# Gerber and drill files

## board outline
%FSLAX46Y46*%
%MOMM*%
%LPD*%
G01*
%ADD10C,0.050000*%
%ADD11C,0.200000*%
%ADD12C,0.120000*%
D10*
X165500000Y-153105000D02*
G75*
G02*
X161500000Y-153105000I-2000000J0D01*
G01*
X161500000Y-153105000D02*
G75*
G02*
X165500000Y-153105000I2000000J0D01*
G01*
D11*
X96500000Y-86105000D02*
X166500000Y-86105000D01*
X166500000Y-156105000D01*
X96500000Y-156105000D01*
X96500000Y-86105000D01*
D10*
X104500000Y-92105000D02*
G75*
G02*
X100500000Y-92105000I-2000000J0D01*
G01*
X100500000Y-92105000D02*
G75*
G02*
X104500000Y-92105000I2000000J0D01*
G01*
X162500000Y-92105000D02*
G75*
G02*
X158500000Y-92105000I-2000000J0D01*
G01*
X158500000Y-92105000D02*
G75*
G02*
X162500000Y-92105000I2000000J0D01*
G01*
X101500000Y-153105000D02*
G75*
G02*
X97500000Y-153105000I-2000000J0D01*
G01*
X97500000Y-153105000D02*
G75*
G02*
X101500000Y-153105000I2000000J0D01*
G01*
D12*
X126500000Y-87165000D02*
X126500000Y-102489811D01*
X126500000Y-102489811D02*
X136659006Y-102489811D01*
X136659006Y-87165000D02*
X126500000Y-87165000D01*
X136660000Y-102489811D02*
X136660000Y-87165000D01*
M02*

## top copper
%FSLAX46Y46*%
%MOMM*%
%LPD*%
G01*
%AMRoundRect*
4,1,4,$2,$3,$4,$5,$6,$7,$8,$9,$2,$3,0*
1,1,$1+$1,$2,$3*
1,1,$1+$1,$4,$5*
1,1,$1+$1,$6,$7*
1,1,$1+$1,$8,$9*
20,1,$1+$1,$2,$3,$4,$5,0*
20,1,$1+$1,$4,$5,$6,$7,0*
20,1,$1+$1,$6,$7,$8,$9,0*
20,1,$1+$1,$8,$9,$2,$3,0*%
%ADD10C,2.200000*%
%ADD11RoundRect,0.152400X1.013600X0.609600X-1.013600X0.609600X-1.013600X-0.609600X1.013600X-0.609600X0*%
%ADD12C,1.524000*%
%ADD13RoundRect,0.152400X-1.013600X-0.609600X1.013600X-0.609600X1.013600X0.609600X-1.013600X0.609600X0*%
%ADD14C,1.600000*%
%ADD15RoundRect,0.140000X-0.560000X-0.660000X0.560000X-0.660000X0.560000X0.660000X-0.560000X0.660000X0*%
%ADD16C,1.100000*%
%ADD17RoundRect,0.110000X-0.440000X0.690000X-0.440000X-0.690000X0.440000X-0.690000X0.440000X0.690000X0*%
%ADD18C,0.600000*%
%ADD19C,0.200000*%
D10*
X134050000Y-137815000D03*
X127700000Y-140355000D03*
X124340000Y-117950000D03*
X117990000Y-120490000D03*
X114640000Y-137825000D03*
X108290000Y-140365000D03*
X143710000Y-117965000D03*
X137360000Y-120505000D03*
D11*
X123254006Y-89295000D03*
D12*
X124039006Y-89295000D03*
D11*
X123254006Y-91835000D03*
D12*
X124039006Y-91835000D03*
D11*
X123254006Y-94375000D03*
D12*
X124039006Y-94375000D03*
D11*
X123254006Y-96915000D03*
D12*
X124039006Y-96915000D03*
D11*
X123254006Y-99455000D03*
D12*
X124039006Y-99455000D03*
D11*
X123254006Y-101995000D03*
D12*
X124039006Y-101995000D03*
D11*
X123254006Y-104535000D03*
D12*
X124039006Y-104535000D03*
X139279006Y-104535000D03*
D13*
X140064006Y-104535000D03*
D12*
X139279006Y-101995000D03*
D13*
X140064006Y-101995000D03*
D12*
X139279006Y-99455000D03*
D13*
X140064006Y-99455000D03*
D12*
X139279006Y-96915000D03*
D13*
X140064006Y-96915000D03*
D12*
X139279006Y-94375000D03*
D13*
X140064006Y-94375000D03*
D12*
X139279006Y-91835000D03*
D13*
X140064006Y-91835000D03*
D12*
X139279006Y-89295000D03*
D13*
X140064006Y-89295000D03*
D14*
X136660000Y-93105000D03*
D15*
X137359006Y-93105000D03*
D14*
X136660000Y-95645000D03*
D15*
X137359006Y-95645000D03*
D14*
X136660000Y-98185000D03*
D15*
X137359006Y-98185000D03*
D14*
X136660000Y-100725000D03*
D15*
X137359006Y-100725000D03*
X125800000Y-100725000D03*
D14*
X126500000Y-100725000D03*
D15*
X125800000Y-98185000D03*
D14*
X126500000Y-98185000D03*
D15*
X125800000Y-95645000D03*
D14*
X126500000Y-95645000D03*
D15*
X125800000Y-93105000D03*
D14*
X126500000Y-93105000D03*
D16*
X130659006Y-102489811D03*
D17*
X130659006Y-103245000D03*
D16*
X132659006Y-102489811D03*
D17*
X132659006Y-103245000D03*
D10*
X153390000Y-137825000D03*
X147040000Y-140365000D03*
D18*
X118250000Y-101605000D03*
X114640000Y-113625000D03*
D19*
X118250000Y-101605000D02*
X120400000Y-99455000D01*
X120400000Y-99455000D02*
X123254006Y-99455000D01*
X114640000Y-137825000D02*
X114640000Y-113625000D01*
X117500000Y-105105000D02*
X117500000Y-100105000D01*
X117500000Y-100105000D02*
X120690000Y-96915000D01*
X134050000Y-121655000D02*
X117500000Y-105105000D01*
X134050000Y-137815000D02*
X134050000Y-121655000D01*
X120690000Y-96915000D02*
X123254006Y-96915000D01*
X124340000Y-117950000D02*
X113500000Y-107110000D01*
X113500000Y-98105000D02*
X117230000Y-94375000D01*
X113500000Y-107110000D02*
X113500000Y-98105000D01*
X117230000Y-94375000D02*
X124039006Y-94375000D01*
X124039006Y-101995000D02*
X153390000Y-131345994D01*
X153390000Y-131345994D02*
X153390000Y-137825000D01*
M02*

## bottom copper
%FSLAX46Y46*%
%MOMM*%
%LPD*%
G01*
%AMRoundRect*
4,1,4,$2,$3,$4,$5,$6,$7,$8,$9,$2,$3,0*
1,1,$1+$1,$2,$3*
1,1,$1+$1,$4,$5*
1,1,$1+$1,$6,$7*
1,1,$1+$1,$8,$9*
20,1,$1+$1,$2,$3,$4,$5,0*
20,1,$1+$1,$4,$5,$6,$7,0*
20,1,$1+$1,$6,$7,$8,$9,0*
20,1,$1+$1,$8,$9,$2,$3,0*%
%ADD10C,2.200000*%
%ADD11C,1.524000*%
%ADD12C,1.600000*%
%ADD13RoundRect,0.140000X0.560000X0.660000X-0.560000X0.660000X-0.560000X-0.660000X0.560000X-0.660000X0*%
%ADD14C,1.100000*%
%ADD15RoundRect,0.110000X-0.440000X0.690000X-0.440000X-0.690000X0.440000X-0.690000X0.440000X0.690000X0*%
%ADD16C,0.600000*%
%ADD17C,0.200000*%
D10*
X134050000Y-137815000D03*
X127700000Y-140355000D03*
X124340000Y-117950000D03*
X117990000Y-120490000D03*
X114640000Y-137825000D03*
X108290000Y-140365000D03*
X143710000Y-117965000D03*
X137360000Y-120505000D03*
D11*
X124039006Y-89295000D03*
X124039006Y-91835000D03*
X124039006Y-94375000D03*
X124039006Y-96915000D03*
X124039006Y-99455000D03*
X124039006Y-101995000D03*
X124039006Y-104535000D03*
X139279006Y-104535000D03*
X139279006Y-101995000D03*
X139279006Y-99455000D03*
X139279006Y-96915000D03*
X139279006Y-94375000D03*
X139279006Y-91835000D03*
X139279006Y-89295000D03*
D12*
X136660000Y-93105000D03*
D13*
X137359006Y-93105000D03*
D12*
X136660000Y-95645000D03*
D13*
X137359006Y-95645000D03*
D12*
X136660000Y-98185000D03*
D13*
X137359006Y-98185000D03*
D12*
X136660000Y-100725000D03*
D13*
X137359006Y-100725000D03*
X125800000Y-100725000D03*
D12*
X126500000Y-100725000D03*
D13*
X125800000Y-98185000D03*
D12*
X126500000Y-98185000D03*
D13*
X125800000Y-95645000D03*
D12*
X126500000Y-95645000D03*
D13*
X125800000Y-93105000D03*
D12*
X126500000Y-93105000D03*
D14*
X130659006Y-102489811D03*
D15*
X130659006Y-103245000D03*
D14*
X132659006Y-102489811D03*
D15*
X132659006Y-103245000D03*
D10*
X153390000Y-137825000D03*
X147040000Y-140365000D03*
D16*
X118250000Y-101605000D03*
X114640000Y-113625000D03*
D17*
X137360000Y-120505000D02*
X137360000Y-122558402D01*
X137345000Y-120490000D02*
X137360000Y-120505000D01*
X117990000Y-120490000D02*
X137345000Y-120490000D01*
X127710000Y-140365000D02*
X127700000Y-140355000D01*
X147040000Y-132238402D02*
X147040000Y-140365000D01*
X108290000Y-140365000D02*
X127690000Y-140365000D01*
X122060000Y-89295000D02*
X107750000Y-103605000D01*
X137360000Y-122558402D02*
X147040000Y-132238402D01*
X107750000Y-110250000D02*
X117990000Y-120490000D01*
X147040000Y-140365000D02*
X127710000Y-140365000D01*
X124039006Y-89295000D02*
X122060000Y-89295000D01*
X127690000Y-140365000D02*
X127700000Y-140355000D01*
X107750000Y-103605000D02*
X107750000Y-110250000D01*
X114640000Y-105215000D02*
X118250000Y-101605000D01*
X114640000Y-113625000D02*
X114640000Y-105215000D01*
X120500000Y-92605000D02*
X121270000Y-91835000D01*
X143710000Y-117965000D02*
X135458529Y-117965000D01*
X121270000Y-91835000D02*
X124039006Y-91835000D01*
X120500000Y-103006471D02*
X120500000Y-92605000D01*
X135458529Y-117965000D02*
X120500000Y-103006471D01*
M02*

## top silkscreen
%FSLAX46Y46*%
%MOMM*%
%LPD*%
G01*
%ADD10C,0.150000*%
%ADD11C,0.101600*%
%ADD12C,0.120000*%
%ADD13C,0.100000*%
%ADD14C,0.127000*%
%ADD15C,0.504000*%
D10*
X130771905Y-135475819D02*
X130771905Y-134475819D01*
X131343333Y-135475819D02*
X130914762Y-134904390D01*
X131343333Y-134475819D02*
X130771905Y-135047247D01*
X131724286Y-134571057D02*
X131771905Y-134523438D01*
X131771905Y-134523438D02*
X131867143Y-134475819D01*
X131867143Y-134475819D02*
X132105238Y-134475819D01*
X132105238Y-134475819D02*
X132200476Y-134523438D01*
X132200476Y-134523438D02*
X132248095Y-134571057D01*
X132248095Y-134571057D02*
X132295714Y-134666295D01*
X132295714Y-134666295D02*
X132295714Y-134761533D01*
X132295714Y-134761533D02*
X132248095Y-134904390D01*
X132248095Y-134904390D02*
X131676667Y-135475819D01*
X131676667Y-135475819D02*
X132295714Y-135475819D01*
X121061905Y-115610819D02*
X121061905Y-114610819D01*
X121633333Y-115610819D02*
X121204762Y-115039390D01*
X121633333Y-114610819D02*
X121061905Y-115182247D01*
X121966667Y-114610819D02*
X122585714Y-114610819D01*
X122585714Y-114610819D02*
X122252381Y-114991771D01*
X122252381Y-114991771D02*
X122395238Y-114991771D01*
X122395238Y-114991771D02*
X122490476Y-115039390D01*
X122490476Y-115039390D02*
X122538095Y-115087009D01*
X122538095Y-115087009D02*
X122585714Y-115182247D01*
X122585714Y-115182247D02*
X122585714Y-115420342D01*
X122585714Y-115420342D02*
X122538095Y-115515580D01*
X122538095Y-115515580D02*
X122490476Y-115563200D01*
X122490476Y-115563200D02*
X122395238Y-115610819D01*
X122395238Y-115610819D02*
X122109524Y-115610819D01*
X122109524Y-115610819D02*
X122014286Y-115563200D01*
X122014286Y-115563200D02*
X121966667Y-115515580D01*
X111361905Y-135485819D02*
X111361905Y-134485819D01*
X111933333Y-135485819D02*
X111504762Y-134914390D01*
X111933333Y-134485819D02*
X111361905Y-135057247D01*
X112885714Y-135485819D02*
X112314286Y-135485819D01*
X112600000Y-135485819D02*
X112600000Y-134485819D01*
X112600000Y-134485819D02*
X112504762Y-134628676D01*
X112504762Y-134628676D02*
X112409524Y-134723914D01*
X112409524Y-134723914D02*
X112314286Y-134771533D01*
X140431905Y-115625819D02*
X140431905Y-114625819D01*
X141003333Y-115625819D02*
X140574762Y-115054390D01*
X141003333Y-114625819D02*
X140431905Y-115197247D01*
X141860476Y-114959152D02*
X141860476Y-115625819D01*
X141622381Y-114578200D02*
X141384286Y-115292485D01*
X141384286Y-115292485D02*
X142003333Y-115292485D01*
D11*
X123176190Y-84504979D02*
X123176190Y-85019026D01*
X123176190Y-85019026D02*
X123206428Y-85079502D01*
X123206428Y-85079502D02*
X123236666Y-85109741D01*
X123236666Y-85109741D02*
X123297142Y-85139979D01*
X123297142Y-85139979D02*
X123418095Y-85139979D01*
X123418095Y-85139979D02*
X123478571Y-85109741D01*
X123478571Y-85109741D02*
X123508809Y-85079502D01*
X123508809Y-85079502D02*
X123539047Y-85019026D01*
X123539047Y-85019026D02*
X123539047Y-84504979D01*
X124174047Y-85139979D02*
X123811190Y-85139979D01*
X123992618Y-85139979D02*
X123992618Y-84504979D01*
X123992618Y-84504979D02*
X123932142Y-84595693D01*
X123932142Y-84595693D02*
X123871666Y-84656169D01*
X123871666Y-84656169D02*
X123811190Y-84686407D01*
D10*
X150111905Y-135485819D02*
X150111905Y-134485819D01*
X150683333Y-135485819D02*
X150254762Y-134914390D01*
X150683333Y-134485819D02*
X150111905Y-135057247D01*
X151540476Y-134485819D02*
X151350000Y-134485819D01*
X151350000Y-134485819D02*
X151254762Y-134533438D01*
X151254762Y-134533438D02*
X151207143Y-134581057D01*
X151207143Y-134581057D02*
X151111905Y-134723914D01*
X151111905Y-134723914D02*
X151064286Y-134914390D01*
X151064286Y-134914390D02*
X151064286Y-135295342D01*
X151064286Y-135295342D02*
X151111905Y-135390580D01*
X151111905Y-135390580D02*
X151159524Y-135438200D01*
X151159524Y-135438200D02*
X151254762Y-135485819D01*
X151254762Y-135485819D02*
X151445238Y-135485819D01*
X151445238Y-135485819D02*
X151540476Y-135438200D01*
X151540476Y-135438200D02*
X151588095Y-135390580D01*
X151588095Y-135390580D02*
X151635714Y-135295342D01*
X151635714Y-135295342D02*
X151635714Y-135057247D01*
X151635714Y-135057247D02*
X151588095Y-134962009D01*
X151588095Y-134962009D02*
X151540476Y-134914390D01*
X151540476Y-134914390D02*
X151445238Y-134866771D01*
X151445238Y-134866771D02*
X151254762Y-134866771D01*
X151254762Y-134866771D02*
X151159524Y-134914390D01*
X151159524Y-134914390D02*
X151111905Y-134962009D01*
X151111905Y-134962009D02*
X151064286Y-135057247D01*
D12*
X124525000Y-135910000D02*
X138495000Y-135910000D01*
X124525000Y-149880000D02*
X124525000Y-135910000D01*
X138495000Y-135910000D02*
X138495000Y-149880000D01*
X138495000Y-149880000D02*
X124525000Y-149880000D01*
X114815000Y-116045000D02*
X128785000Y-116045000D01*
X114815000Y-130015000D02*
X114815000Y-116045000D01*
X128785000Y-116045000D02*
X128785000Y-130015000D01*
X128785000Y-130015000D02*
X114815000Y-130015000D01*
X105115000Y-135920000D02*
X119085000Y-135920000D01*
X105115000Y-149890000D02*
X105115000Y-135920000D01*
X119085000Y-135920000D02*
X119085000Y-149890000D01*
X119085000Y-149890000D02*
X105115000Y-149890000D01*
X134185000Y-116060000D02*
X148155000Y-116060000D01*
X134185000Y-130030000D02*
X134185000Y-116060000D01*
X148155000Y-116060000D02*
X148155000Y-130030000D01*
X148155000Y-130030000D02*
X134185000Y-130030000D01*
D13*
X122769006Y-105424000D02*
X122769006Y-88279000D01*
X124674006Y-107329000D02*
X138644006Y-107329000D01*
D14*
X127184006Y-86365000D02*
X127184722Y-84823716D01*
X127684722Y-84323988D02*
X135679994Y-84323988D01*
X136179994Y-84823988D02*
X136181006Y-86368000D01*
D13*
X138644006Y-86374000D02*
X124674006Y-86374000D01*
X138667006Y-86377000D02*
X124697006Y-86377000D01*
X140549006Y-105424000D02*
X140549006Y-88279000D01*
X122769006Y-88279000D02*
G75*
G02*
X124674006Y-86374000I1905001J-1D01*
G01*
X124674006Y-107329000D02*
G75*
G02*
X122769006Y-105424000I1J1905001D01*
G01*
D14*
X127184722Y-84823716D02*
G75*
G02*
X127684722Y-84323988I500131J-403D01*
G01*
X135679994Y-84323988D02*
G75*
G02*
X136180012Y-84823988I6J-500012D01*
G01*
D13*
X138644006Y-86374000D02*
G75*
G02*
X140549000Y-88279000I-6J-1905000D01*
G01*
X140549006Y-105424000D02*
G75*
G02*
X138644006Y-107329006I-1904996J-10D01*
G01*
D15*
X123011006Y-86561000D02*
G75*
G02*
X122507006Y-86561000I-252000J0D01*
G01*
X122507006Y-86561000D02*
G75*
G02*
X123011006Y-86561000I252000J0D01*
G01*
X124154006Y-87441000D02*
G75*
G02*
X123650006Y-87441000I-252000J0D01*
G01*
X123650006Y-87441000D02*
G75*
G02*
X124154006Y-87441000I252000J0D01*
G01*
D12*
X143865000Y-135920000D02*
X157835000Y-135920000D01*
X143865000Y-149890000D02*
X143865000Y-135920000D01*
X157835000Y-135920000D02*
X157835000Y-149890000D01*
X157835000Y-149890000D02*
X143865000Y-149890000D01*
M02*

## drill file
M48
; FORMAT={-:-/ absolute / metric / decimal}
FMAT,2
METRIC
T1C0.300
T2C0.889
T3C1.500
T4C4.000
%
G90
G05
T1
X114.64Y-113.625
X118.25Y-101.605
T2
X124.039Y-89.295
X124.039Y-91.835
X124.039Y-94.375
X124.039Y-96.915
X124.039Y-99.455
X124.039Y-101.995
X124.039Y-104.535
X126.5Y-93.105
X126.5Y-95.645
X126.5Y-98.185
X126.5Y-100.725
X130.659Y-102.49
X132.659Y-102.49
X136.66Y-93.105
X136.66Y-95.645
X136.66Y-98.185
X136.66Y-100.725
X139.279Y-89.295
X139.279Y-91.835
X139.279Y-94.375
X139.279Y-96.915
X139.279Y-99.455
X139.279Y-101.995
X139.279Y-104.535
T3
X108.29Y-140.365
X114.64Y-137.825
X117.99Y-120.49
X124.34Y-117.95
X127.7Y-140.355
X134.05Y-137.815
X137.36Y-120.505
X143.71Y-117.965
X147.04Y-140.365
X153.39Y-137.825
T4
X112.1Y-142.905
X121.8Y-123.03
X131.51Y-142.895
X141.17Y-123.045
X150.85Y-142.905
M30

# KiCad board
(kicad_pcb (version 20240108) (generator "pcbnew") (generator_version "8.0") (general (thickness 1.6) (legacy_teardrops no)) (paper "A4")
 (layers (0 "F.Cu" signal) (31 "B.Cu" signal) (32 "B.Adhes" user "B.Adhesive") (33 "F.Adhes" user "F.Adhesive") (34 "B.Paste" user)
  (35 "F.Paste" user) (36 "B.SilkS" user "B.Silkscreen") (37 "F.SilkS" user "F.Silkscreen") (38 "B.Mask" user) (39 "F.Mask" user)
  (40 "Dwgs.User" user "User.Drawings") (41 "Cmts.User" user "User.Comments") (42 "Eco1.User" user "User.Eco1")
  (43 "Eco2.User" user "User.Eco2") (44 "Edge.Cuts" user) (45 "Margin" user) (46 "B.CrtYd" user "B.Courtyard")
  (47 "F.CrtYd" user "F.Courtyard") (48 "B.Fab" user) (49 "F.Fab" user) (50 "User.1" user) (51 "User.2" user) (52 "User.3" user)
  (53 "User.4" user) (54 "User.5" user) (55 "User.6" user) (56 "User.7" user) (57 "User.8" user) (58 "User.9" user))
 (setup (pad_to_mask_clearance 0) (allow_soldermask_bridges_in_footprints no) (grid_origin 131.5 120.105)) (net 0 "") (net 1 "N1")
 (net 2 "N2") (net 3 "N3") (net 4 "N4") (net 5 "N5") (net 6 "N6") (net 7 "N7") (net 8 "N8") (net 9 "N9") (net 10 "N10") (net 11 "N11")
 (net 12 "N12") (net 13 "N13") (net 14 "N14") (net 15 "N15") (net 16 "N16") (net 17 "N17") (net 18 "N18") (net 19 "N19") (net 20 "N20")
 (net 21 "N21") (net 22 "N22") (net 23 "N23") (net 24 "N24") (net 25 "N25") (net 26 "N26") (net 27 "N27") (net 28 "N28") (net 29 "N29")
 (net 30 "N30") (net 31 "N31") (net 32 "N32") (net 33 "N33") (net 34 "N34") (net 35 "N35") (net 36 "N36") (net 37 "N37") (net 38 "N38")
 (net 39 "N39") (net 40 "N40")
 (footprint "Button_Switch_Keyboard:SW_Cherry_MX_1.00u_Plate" (layer "F.Cu") (at 134.05 137.815)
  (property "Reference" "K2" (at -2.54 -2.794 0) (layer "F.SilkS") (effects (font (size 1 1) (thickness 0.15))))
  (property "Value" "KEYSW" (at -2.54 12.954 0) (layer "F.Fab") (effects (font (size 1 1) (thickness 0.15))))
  (fp_line (start -9.525 -1.905) (end 4.445 -1.905) (stroke (width 0.12) (type solid)) (layer "F.SilkS"))
  (fp_line (start -9.525 12.065) (end -9.525 -1.905) (stroke (width 0.12) (type solid)) (layer "F.SilkS"))
  (fp_line (start 4.445 -1.905) (end 4.445 12.065) (stroke (width 0.12) (type solid)) (layer "F.SilkS"))
  (fp_line (start 4.445 12.065) (end -9.525 12.065) (stroke (width 0.12) (type solid)) (layer "F.SilkS"))
  (pad "" np_thru_hole circle (at -2.54 5.08) (size 4 4) (drill 4) (layers "*.Cu" "*.Mask"))
  (pad "1" thru_hole circle (at 0 0) (size 2.2 2.2) (drill 1.5) (layers "*.Cu" "*.Mask") (remove_unused_layers no) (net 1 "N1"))
  (pad "2" thru_hole circle (at -6.35 2.54) (size 2.2 2.2) (drill 1.5) (layers "*.Cu" "*.Mask") (remove_unused_layers no) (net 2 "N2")))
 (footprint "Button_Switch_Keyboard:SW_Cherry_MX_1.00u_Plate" (layer "F.Cu") (at 124.34 117.95)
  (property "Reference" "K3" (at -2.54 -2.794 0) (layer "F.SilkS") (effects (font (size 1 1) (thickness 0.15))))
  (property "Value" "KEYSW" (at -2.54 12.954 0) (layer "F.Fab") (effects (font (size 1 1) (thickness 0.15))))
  (fp_line (start -9.525 -1.905) (end 4.445 -1.905) (stroke (width 0.12) (type solid)) (layer "F.SilkS"))
  (fp_line (start -9.525 12.065) (end -9.525 -1.905) (stroke (width 0.12) (type solid)) (layer "F.SilkS"))
  (fp_line (start 4.445 -1.905) (end 4.445 12.065) (stroke (width 0.12) (type solid)) (layer "F.SilkS"))
  (fp_line (start 4.445 12.065) (end -9.525 12.065) (stroke (width 0.12) (type solid)) (layer "F.SilkS"))
  (pad "" np_thru_hole circle (at -2.54 5.08) (size 4 4) (drill 4) (layers "*.Cu" "*.Mask"))
  (pad "1" thru_hole circle (at 0 0) (size 2.2 2.2) (drill 1.5) (layers "*.Cu" "*.Mask") (remove_unused_layers no) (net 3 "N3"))
  (pad "2" thru_hole circle (at -6.35 2.54) (size 2.2 2.2) (drill 1.5) (layers "*.Cu" "*.Mask") (remove_unused_layers no) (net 2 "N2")))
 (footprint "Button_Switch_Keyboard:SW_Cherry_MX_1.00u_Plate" (layer "F.Cu") (at 114.64 137.825)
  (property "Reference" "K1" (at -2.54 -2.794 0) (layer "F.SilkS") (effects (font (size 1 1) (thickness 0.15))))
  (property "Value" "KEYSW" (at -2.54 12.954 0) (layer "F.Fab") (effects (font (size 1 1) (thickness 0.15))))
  (fp_line (start -9.525 -1.905) (end 4.445 -1.905) (stroke (width 0.12) (type solid)) (layer "F.SilkS"))
  (fp_line (start -9.525 12.065) (end -9.525 -1.905) (stroke (width 0.12) (type solid)) (layer "F.SilkS"))
  (fp_line (start 4.445 -1.905) (end 4.445 12.065) (stroke (width 0.12) (type solid)) (layer "F.SilkS"))
  (fp_line (start 4.445 12.065) (end -9.525 12.065) (stroke (width 0.12) (type solid)) (layer "F.SilkS"))
  (pad "" np_thru_hole circle (at -2.54 5.08) (size 4 4) (drill 4) (layers "*.Cu" "*.Mask"))
  (pad "1" thru_hole circle (at 0 0) (size 2.2 2.2) (drill 1.5) (layers "*.Cu" "*.Mask") (remove_unused_layers no) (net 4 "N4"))
  (pad "2" thru_hole circle (at -6.35 2.54) (size 2.2 2.2) (drill 1.5) (layers "*.Cu" "*.Mask") (remove_unused_layers no) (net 2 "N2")))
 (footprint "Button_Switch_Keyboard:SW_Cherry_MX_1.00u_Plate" (layer "F.Cu") (at 143.71 117.965)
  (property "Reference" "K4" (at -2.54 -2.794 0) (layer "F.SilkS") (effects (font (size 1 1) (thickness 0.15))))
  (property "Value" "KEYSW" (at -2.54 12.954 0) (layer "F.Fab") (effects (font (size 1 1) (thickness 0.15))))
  (fp_line (start -9.525 -1.905) (end 4.445 -1.905) (stroke (width 0.12) (type solid)) (layer "F.SilkS"))
  (fp_line (start -9.525 12.065) (end -9.525 -1.905) (stroke (width 0.12) (type solid)) (layer "F.SilkS"))
  (fp_line (start 4.445 -1.905) (end 4.445 12.065) (stroke (width 0.12) (type solid)) (layer "F.SilkS"))
  (fp_line (start 4.445 12.065) (end -9.525 12.065) (stroke (width 0.12) (type solid)) (layer "F.SilkS"))
  (pad "" np_thru_hole circle (at -2.54 5.08) (size 4 4) (drill 4) (layers "*.Cu" "*.Mask"))
  (pad "1" thru_hole circle (at 0 0) (size 2.2 2.2) (drill 1.5) (layers "*.Cu" "*.Mask") (remove_unused_layers no) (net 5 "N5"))
  (pad "2" thru_hole circle (at -6.35 2.54) (size 2.2 2.2) (drill 1.5) (layers "*.Cu" "*.Mask") (remove_unused_layers no) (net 2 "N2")))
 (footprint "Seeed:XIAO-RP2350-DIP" (layer "F.Cu") (at 131.66 96.8515)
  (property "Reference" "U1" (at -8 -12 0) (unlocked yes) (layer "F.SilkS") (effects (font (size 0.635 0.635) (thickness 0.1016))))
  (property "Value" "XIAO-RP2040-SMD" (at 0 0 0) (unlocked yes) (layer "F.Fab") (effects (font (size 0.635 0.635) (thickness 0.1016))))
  (fp_line (start -8.890994 8.5725) (end -8.890994 -8.5725) (stroke (width 0.1) (type solid)) (layer "F.SilkS"))
  (fp_line (start -6.985994 10.4775) (end 6.984006 10.4775) (stroke (width 0.1) (type solid)) (layer "F.SilkS"))
  (fp_line (start -4.475994 -10.4865) (end -4.475278 -12.027784) (stroke (width 0.127) (type solid)) (layer "F.SilkS"))
  (fp_line (start -3.975278 -12.527512) (end 4.019994 -12.527512) (stroke (width 0.127) (type solid)) (layer "F.SilkS"))
  (fp_line (start 4.519994 -12.027512) (end 4.521006 -10.4835) (stroke (width 0.127) (type solid)) (layer "F.SilkS"))
  (fp_line (start 6.984006 -10.4775) (end -6.985994 -10.4775) (stroke (width 0.1) (type solid)) (layer "F.SilkS"))
  (fp_line (start 7.007006 -10.4745) (end -6.962994 -10.4745) (stroke (width 0.1) (type solid)) (layer "F.SilkS"))
  (fp_line (start 8.889006 8.5725) (end 8.889006 -8.5725) (stroke (width 0.1) (type solid)) (layer "F.SilkS"))
  (fp_arc (start -8.890994 -8.5725) (mid -8.333032 -9.919538) (end -6.985994 -10.4775) (stroke (width 0.1) (type solid)) (layer "F.SilkS"))
  (fp_arc (start -6.985994 10.4775) (mid -8.333032 9.919538) (end -8.890994 8.5725) (stroke (width 0.1) (type solid)) (layer "F.SilkS"))
  (fp_arc (start -4.475278 -12.027784) (mid -4.328697 -12.381123) (end -3.975278 -12.527512) (stroke (width 0.127) (type default))
   (layer "F.SilkS"))
  (fp_arc (start 4.019994 -12.527512) (mid 4.373556 -12.381068) (end 4.519994 -12.027512) (stroke (width 0.127) (type default))
   (layer "F.SilkS"))
  (fp_arc (start 6.984006 -10.4775) (mid 8.331041 -9.919536) (end 8.889006 -8.5725) (stroke (width 0.1) (type solid)) (layer "F.SilkS"))
  (fp_arc (start 8.889006 8.5725) (mid 8.331047 9.91954) (end 6.984006 10.4775) (stroke (width 0.1) (type solid)) (layer "F.SilkS"))
  (fp_circle (center -8.900994 -10.2905) (end -8.900994 -10.5445) (stroke (width 0.5) (type solid)) (fill solid) (layer "F.SilkS"))
  (fp_circle (center -7.757994 -9.4105) (end -7.757994 -9.6645) (stroke (width 0.5) (type solid)) (fill solid) (layer "F.SilkS"))
  (fp_line (start -5.16 -9.6865) (end -5.16 5.638311) (stroke (width 0.12) (type default)) (layer "Edge.Cuts"))
  (fp_line (start -5.16 5.638311) (end 4.999006 5.638311) (stroke (width 0.12) (type default)) (layer "Edge.Cuts"))
  (fp_line (start 4.999006 -9.6865) (end -5.16 -9.6865) (stroke (width 0.12) (type default)) (layer "Edge.Cuts"))
  (fp_line (start 5 5.638311) (end 5 -9.6865) (stroke (width 0.12) (type default)) (layer "Edge.Cuts"))
  (pad "1" smd roundrect (at -8.405994 -7.5565 180) (size 2.332 1.524) (layers "F.Cu" "F.Mask") (roundrect_rratio 0.1) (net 2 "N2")
   (thermal_bridge_angle 45))
  (pad "1" thru_hole circle (at -7.620994 -7.5565 180) (size 1.524 1.524) (drill 0.889) (layers "*.Cu" "*.Mask") (remove_unused_layers no)
   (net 2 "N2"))
  (pad "2" smd roundrect (at -8.405994 -5.0165 180) (size 2.332 1.524) (layers "F.Cu" "F.Mask") (roundrect_rratio 0.1) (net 5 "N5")
   (thermal_bridge_angle 45))
  (pad "2" thru_hole circle (at -7.620994 -5.0165 180) (size 1.524 1.524) (drill 0.889) (layers "*.Cu" "*.Mask") (remove_unused_layers no)
   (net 5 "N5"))
  (pad "3" smd roundrect (at -8.405994 -2.4765 180) (size 2.332 1.524) (layers "F.Cu" "F.Mask") (roundrect_rratio 0.1) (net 3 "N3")
   (thermal_bridge_angle 45))
  (pad "3" thru_hole circle (at -7.620994 -2.4765 180) (size 1.524 1.524) (drill 0.889) (layers "*.Cu" "*.Mask") (remove_unused_layers no)
   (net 3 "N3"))
  (pad "4" smd roundrect (at -8.405994 0.0635 180) (size 2.332 1.524) (layers "F.Cu" "F.Mask") (roundrect_rratio 0.1) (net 1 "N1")
   (thermal_bridge_angle 45))
  (pad "4" thru_hole circle (at -7.620994 0.0635 180) (size 1.524 1.524) (drill 0.889) (layers "*.Cu" "*.Mask") (remove_unused_layers no)
   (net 1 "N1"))
  (pad "5" smd roundrect (at -8.405994 2.6035 180) (size 2.332 1.524) (layers "F.Cu" "F.Mask") (roundrect_rratio 0.1) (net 4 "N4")
   (thermal_bridge_angle 45))
  (pad "5" thru_hole circle (at -7.620994 2.6035 180) (size 1.524 1.524) (drill 0.889) (layers "*.Cu" "*.Mask") (remove_unused_layers no)
   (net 4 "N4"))
  (pad "6" smd roundrect (at -8.405994 5.1435 180) (size 2.332 1.524) (layers "F.Cu" "F.Mask") (roundrect_rratio 0.1) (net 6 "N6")
   (thermal_bridge_angle 45))
  (pad "6" thru_hole circle (at -7.620994 5.1435 180) (size 1.524 1.524) (drill 0.889) (layers "*.Cu" "*.Mask") (remove_unused_layers no)
   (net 6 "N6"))
  (pad "7" smd roundrect (at -8.405994 7.6835 180) (size 2.332 1.524) (layers "F.Cu" "F.Mask") (roundrect_rratio 0.1) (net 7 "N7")
   (thermal_bridge_angle 45))
  (pad "7" thru_hole circle (at -7.620994 7.6835 180) (size 1.524 1.524) (drill 0.889) (layers "*.Cu" "*.Mask") (remove_unused_layers no)
   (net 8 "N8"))
  (pad "8" thru_hole circle (at 7.619006 7.6835) (size 1.524 1.524) (drill 0.889) (layers "*.Cu" "*.Mask") (remove_unused_layers no)
   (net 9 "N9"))
  (pad "8" smd roundrect (at 8.404006 7.6835) (size 2.332 1.524) (layers "F.Cu" "F.Mask") (roundrect_rratio 0.1) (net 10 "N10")
   (thermal_bridge_angle 45))
  (pad "9" thru_hole circle (at 7.619006 5.1435) (size 1.524 1.524) (drill 0.889) (layers "*.Cu" "*.Mask") (remove_unused_layers no)
   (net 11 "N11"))
  (pad "9" smd roundrect (at 8.404006 5.1435) (size 2.332 1.524) (layers "F.Cu" "F.Mask") (roundrect_rratio 0.1) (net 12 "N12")
   (thermal_bridge_angle 45))
  (pad "10" thru_hole circle (at 7.619006 2.6035) (size 1.524 1.524) (drill 0.889) (layers "*.Cu" "*.Mask") (remove_unused_layers no)
   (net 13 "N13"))
  (pad "10" smd roundrect (at 8.404006 2.6035) (size 2.332 1.524) (layers "F.Cu" "F.Mask") (roundrect_rratio 0.1) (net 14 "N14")
   (thermal_bridge_angle 45))
  (pad "11" thru_hole circle (at 7.619006 0.0635) (size 1.524 1.524) (drill 0.889) (layers "*.Cu" "*.Mask") (remove_unused_layers no)
   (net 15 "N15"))
  (pad "11" smd roundrect (at 8.404006 0.0635) (size 2.332 1.524) (layers "F.Cu" "F.Mask") (roundrect_rratio 0.1) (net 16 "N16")
   (thermal_bridge_angle 45))
  (pad "12" thru_hole circle (at 7.619006 -2.4765) (size 1.524 1.524) (drill 0.889) (layers "*.Cu" "*.Mask") (remove_unused_layers no)
   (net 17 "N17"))
  (pad "12" smd roundrect (at 8.404006 -2.4765) (size 2.332 1.524) (layers "F.Cu" "F.Mask") (roundrect_rratio 0.1) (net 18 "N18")
   (thermal_bridge_angle 45))
  (pad "13" thru_hole circle (at 7.619006 -5.0165) (size 1.524 1.524) (drill 0.889) (layers "*.Cu" "*.Mask") (remove_unused_layers no)
   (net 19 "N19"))
  (pad "13" smd roundrect (at 8.404006 -5.0165) (size 2.332 1.524) (layers "F.Cu" "F.Mask") (roundrect_rratio 0.1) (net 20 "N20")
   (thermal_bridge_angle 45))
  (pad "14" thru_hole circle (at 7.619006 -7.5565) (size 1.524 1.524) (drill 0.889) (layers "*.Cu" "*.Mask") (remove_unused_layers no)
   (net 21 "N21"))
  (pad "14" smd roundrect (at 8.404006 -7.5565) (size 2.332 1.524) (layers "F.Cu" "F.Mask") (roundrect_rratio 0.1) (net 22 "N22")
   (thermal_bridge_angle 45))
  (pad "15" thru_hole circle (at 5 -3.7465 180) (size 1.6 1.6) (drill 0.889) (layers "*.Cu" "*.Mask") (remove_unused_layers no)
   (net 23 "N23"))
  (pad "15" smd roundrect (at 5.699006 -3.7465) (size 1.4 1.6) (layers "F.Cu" "F.Mask") (roundrect_rratio 0.1) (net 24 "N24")
   (thermal_bridge_angle 45))
  (pad "15" smd roundrect (at 5.699006 -3.7465 180) (size 1.4 1.6) (layers "B.Cu" "B.Paste" "B.Mask") (roundrect_rratio 0.1) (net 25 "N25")
   (thermal_bridge_angle 45))
  (pad "16" thru_hole circle (at 5 -1.2065 180) (size 1.6 1.6) (drill 0.889) (layers "*.Cu" "*.Mask") (remove_unused_layers no)
   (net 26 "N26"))
  (pad "16" smd roundrect (at 5.699006 -1.2065) (size 1.4 1.6) (layers "F.Cu" "F.Mask") (roundrect_rratio 0.1) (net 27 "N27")
   (thermal_bridge_angle 45))
  (pad "16" smd roundrect (at 5.699006 -1.2065 180) (size 1.4 1.6) (layers "B.Cu" "B.Paste" "B.Mask") (roundrect_rratio 0.1) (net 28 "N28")
   (thermal_bridge_angle 45))
  (pad "17" thru_hole circle (at 5 1.3335 180) (size 1.6 1.6) (drill 0.889) (layers "*.Cu" "*.Mask") (remove_unused_layers no)
   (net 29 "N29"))
  (pad "17" smd roundrect (at 5.699006 1.3335) (size 1.4 1.6) (layers "F.Cu" "F.Mask") (roundrect_rratio 0.1) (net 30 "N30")
   (thermal_bridge_angle 45))
  (pad "17" smd roundrect (at 5.699006 1.3335 180) (size 1.4 1.6) (layers "B.Cu" "B.Paste" "B.Mask") (roundrect_rratio 0.1) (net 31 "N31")
   (thermal_bridge_angle 45))
  (pad "18" thru_hole circle (at 5 3.8735 180) (size 1.6 1.6) (drill 0.889) (layers "*.Cu" "*.Mask") (remove_unused_layers no)
   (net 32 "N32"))
  (pad "18" smd roundrect (at 5.699006 3.8735) (size 1.4 1.6) (layers "F.Cu" "F.Mask") (roundrect_rratio 0.1) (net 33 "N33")
   (thermal_bridge_angle 45))
  (pad "18" smd roundrect (at 5.699006 3.8735 180) (size 1.4 1.6) (layers "B.Cu" "B.Paste" "B.Mask") (roundrect_rratio 0.1) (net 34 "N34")
   (thermal_bridge_angle 45))
  (pad "19" smd roundrect (at -5.86 3.8735) (size 1.4 1.6) (layers "F.Cu" "F.Mask") (roundrect_rratio 0.1) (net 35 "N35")
   (thermal_bridge_angle 45))
  (pad "19" smd roundrect (at -5.86 3.8735 180) (size 1.4 1.6) (layers "B.Cu" "B.Paste" "B.Mask") (roundrect_rratio 0.1) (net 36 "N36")
   (thermal_bridge_angle 45))
  (pad "19" thru_hole circle (at -5.16 3.8735 180) (size 1.6 1.6) (drill 0.889) (layers "*.Cu" "*.Mask") (remove_unused_layers no)
   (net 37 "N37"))
  (pad "20" smd roundrect (at -5.86 1.3335) (size 1.4 1.6) (layers "F.Cu" "F.Mask") (roundrect_rratio 0.1) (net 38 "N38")
   (thermal_bridge_angle 45))
  (pad "20" smd roundrect (at -5.86 1.3335 180) (size 1.4 1.6) (layers "B.Cu" "B.Paste" "B.Mask") (roundrect_rratio 0.1) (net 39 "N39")
   (thermal_bridge_angle 45))
  (pad "20" thru_hole circle (at -5.16 1.3335 180) (size 1.6 1.6) (drill 0.889) (layers "*.Cu" "*.Mask") (remove_unused_layers no)
   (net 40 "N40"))
  (pad "21" smd roundrect (at -5.86 -1.2065) (size 1.4 1.6) (layers "F.Cu" "F.Mask") (roundrect_rratio 0.1) (thermal_bridge_angle 45))
  (pad "21" smd roundrect (at -5.86 -1.2065 180) (size 1.4 1.6) (layers "B.Cu" "B.Paste" "B.Mask") (roundrect_rratio 0.1)
   (thermal_bridge_angle 45))
  (pad "21" thru_hole circle (at -5.16 -1.2065 180) (size 1.6 1.6) (drill 0.889) (layers "*.Cu" "*.Mask") (remove_unused_layers no))
  (pad "22" smd roundrect (at -5.86 -3.7465) (size 1.4 1.6) (layers "F.Cu" "F.Mask") (roundrect_rratio 0.1) (thermal_bridge_angle 45))
  (pad "22" smd roundrect (at -5.86 -3.7465 180) (size 1.4 1.6) (layers "B.Cu" "B.Paste" "B.Mask") (roundrect_rratio 0.1)
   (thermal_bridge_angle 45))
  (pad "22" thru_hole circle (at -5.16 -3.7465 180) (size 1.6 1.6) (drill 0.889) (layers "*.Cu" "*.Mask") (remove_unused_layers no))
  (pad "23" thru_hole circle (at -1.000994 5.638311 180) (size 1.1 1.1) (drill 0.889) (layers "*.Cu" "*.Mask") (remove_unused_layers no))
  (pad "23" smd roundrect (at -1.000994 6.3935 270) (size 1.6 1.1) (layers "F.Cu" "F.Mask") (roundrect_rratio 0.1) (thermal_bridge_angle 45))
  (pad "23" smd roundrect (at -1.000994 6.3935 270) (size 1.6 1.1) (layers "B.Cu" "B.Paste" "B.Mask") (roundrect_rratio 0.1)
   (thermal_bridge_angle 45))
  (pad "24" thru_hole circle (at 0.999006 5.638311 180) (size 1.1 1.1) (drill 0.889) (layers "*.Cu" "*.Mask") (remove_unused_layers no))
  (pad "24" smd roundrect (at 0.999006 6.3935 270) (size 1.6 1.1) (layers "F.Cu" "F.Mask") (roundrect_rratio 0.1) (thermal_bridge_angle 45))
  (pad "24" smd roundrect (at 0.999006 6.3935 270) (size 1.6 1.1) (layers "B.Cu" "B.Paste" "B.Mask") (roundrect_rratio 0.1)
   (thermal_bridge_angle 45)))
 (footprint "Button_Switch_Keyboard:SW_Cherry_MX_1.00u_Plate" (layer "F.Cu") (at 153.39 137.825)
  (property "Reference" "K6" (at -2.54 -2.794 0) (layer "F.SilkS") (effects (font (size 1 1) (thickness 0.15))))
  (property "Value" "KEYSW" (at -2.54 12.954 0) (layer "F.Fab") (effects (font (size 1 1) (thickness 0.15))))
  (fp_line (start -9.525 -1.905) (end 4.445 -1.905) (stroke (width 0.12) (type solid)) (layer "F.SilkS"))
  (fp_line (start -9.525 12.065) (end -9.525 -1.905) (stroke (width 0.12) (type solid)) (layer "F.SilkS"))
  (fp_line (start 4.445 -1.905) (end 4.445 12.065) (stroke (width 0.12) (type solid)) (layer "F.SilkS"))
  (fp_line (start 4.445 12.065) (end -9.525 12.065) (stroke (width 0.12) (type solid)) (layer "F.SilkS"))
  (pad "" np_thru_hole circle (at -2.54 5.08) (size 4 4) (drill 4) (layers "*.Cu" "*.Mask"))
  (pad "1" thru_hole circle (at 0 0) (size 2.2 2.2) (drill 1.5) (layers "*.Cu" "*.Mask") (remove_unused_layers no) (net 6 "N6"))
  (pad "2" thru_hole circle (at -6.35 2.54) (size 2.2 2.2) (drill 1.5) (layers "*.Cu" "*.Mask") (remove_unused_layers no) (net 2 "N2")))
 (gr_circle (center 163.5 153.105) (end 165.5 153.105) (stroke (width 0.05) (type default)) (fill none) (layer "Edge.Cuts"))
 (gr_rect (start 96.5 86.105) (end 166.5 156.105) (stroke (width 0.2) (type default)) (fill none) (layer "Edge.Cuts"))
 (gr_circle (center 102.5 92.105) (end 104.5 92.105) (stroke (width 0.05) (type default)) (fill none) (layer "Edge.Cuts"))
 (gr_circle (center 160.5 92.105) (end 162.5 92.105) (stroke (width 0.05) (type default)) (fill none) (layer "Edge.Cuts"))
 (gr_circle (center 99.5 153.105) (end 101.5 153.105) (stroke (width 0.05) (type default)) (fill none) (layer "Edge.Cuts"))
 (segment (start 137.36 120.505) (end 137.36 122.558402) (width 0.2) (layer "B.Cu") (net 2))
 (segment (start 137.345 120.49) (end 137.36 120.505) (width 0.2) (layer "B.Cu") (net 2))
 (segment (start 117.99 120.49) (end 137.345 120.49) (width 0.2) (layer "B.Cu") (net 2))
 (segment (start 127.71 140.365) (end 127.7 140.355) (width 0.2) (layer "B.Cu") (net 2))
 (segment (start 147.04 132.238402) (end 147.04 140.365) (width 0.2) (layer "B.Cu") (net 2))
 (segment (start 108.29 140.365) (end 127.69 140.365) (width 0.2) (layer "B.Cu") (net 2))
 (segment (start 122.06 89.295) (end 107.75 103.605) (width 0.2) (layer "B.Cu") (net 2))
 (segment (start 137.36 122.558402) (end 147.04 132.238402) (width 0.2) (layer "B.Cu") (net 2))
 (segment (start 107.75 110.25) (end 117.99 120.49) (width 0.2) (layer "B.Cu") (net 2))
 (segment (start 147.04 140.365) (end 127.71 140.365) (width 0.2) (layer "B.Cu") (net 2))
 (segment (start 124.039006 89.295) (end 122.06 89.295) (width 0.2) (layer "B.Cu") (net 2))
 (segment (start 127.69 140.365) (end 127.7 140.355) (width 0.2) (layer "B.Cu") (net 2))
 (segment (start 107.75 103.605) (end 107.75 110.25) (width 0.2) (layer "B.Cu") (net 2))
 (segment (start 118.25 101.605) (end 120.4 99.455) (width 0.2) (layer "F.Cu") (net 4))
 (segment (start 120.4 99.455) (end 123.254006 99.455) (width 0.2) (layer "F.Cu") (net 4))
 (segment (start 114.64 137.825) (end 114.64 113.625) (width 0.2) (layer "F.Cu") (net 4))
 (via (at 118.25 101.605) (size 0.6) (drill 0.3) (layers "F.Cu" "B.Cu") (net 4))
 (via (at 114.64 113.625) (size 0.6) (drill 0.3) (layers "F.Cu" "B.Cu") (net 4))
 (segment (start 114.64 105.215) (end 118.25 101.605) (width 0.2) (layer "B.Cu") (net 4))
 (segment (start 114.64 113.625) (end 114.64 105.215) (width 0.2) (layer "B.Cu") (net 4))
 (segment (start 117.5 105.105) (end 117.5 100.105) (width 0.2) (layer "F.Cu") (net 1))
 (segment (start 117.5 100.105) (end 120.69 96.915) (width 0.2) (layer "F.Cu") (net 1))
 (segment (start 134.05 121.655) (end 117.5 105.105) (width 0.2) (layer "F.Cu") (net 1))
 (segment (start 134.05 137.815) (end 134.05 121.655) (width 0.2) (layer "F.Cu") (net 1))
 (segment (start 120.69 96.915) (end 123.254006 96.915) (width 0.2) (layer "F.Cu") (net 1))
 (segment (start 124.34 117.95) (end 113.5 107.11) (width 0.2) (layer "F.Cu") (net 3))
 (segment (start 113.5 98.105) (end 117.23 94.375) (width 0.2) (layer "F.Cu") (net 3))
 (segment (start 113.5 107.11) (end 113.5 98.105) (width 0.2) (layer "F.Cu") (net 3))
 (segment (start 117.23 94.375) (end 124.039006 94.375) (width 0.2) (layer "F.Cu") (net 3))
 (segment (start 120.5 92.605) (end 121.27 91.835) (width 0.2) (layer "B.Cu") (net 5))
 (segment (start 143.71 117.965) (end 135.458529 117.965) (width 0.2) (layer "B.Cu") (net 5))
 (segment (start 121.27 91.835) (end 124.039006 91.835) (width 0.2) (layer "B.Cu") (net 5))
 (segment (start 120.5 103.006471) (end 120.5 92.605) (width 0.2) (layer "B.Cu") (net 5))
 (segment (start 135.458529 117.965) (end 120.5 103.006471) (width 0.2) (layer "B.Cu") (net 5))
 (segment (start 124.039006 101.995) (end 153.39 131.345994) (width 0.2) (layer "F.Cu") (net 6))
 (segment (start 153.39 131.345994) (end 153.39 137.825) (width 0.2) (layer "F.Cu") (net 6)))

